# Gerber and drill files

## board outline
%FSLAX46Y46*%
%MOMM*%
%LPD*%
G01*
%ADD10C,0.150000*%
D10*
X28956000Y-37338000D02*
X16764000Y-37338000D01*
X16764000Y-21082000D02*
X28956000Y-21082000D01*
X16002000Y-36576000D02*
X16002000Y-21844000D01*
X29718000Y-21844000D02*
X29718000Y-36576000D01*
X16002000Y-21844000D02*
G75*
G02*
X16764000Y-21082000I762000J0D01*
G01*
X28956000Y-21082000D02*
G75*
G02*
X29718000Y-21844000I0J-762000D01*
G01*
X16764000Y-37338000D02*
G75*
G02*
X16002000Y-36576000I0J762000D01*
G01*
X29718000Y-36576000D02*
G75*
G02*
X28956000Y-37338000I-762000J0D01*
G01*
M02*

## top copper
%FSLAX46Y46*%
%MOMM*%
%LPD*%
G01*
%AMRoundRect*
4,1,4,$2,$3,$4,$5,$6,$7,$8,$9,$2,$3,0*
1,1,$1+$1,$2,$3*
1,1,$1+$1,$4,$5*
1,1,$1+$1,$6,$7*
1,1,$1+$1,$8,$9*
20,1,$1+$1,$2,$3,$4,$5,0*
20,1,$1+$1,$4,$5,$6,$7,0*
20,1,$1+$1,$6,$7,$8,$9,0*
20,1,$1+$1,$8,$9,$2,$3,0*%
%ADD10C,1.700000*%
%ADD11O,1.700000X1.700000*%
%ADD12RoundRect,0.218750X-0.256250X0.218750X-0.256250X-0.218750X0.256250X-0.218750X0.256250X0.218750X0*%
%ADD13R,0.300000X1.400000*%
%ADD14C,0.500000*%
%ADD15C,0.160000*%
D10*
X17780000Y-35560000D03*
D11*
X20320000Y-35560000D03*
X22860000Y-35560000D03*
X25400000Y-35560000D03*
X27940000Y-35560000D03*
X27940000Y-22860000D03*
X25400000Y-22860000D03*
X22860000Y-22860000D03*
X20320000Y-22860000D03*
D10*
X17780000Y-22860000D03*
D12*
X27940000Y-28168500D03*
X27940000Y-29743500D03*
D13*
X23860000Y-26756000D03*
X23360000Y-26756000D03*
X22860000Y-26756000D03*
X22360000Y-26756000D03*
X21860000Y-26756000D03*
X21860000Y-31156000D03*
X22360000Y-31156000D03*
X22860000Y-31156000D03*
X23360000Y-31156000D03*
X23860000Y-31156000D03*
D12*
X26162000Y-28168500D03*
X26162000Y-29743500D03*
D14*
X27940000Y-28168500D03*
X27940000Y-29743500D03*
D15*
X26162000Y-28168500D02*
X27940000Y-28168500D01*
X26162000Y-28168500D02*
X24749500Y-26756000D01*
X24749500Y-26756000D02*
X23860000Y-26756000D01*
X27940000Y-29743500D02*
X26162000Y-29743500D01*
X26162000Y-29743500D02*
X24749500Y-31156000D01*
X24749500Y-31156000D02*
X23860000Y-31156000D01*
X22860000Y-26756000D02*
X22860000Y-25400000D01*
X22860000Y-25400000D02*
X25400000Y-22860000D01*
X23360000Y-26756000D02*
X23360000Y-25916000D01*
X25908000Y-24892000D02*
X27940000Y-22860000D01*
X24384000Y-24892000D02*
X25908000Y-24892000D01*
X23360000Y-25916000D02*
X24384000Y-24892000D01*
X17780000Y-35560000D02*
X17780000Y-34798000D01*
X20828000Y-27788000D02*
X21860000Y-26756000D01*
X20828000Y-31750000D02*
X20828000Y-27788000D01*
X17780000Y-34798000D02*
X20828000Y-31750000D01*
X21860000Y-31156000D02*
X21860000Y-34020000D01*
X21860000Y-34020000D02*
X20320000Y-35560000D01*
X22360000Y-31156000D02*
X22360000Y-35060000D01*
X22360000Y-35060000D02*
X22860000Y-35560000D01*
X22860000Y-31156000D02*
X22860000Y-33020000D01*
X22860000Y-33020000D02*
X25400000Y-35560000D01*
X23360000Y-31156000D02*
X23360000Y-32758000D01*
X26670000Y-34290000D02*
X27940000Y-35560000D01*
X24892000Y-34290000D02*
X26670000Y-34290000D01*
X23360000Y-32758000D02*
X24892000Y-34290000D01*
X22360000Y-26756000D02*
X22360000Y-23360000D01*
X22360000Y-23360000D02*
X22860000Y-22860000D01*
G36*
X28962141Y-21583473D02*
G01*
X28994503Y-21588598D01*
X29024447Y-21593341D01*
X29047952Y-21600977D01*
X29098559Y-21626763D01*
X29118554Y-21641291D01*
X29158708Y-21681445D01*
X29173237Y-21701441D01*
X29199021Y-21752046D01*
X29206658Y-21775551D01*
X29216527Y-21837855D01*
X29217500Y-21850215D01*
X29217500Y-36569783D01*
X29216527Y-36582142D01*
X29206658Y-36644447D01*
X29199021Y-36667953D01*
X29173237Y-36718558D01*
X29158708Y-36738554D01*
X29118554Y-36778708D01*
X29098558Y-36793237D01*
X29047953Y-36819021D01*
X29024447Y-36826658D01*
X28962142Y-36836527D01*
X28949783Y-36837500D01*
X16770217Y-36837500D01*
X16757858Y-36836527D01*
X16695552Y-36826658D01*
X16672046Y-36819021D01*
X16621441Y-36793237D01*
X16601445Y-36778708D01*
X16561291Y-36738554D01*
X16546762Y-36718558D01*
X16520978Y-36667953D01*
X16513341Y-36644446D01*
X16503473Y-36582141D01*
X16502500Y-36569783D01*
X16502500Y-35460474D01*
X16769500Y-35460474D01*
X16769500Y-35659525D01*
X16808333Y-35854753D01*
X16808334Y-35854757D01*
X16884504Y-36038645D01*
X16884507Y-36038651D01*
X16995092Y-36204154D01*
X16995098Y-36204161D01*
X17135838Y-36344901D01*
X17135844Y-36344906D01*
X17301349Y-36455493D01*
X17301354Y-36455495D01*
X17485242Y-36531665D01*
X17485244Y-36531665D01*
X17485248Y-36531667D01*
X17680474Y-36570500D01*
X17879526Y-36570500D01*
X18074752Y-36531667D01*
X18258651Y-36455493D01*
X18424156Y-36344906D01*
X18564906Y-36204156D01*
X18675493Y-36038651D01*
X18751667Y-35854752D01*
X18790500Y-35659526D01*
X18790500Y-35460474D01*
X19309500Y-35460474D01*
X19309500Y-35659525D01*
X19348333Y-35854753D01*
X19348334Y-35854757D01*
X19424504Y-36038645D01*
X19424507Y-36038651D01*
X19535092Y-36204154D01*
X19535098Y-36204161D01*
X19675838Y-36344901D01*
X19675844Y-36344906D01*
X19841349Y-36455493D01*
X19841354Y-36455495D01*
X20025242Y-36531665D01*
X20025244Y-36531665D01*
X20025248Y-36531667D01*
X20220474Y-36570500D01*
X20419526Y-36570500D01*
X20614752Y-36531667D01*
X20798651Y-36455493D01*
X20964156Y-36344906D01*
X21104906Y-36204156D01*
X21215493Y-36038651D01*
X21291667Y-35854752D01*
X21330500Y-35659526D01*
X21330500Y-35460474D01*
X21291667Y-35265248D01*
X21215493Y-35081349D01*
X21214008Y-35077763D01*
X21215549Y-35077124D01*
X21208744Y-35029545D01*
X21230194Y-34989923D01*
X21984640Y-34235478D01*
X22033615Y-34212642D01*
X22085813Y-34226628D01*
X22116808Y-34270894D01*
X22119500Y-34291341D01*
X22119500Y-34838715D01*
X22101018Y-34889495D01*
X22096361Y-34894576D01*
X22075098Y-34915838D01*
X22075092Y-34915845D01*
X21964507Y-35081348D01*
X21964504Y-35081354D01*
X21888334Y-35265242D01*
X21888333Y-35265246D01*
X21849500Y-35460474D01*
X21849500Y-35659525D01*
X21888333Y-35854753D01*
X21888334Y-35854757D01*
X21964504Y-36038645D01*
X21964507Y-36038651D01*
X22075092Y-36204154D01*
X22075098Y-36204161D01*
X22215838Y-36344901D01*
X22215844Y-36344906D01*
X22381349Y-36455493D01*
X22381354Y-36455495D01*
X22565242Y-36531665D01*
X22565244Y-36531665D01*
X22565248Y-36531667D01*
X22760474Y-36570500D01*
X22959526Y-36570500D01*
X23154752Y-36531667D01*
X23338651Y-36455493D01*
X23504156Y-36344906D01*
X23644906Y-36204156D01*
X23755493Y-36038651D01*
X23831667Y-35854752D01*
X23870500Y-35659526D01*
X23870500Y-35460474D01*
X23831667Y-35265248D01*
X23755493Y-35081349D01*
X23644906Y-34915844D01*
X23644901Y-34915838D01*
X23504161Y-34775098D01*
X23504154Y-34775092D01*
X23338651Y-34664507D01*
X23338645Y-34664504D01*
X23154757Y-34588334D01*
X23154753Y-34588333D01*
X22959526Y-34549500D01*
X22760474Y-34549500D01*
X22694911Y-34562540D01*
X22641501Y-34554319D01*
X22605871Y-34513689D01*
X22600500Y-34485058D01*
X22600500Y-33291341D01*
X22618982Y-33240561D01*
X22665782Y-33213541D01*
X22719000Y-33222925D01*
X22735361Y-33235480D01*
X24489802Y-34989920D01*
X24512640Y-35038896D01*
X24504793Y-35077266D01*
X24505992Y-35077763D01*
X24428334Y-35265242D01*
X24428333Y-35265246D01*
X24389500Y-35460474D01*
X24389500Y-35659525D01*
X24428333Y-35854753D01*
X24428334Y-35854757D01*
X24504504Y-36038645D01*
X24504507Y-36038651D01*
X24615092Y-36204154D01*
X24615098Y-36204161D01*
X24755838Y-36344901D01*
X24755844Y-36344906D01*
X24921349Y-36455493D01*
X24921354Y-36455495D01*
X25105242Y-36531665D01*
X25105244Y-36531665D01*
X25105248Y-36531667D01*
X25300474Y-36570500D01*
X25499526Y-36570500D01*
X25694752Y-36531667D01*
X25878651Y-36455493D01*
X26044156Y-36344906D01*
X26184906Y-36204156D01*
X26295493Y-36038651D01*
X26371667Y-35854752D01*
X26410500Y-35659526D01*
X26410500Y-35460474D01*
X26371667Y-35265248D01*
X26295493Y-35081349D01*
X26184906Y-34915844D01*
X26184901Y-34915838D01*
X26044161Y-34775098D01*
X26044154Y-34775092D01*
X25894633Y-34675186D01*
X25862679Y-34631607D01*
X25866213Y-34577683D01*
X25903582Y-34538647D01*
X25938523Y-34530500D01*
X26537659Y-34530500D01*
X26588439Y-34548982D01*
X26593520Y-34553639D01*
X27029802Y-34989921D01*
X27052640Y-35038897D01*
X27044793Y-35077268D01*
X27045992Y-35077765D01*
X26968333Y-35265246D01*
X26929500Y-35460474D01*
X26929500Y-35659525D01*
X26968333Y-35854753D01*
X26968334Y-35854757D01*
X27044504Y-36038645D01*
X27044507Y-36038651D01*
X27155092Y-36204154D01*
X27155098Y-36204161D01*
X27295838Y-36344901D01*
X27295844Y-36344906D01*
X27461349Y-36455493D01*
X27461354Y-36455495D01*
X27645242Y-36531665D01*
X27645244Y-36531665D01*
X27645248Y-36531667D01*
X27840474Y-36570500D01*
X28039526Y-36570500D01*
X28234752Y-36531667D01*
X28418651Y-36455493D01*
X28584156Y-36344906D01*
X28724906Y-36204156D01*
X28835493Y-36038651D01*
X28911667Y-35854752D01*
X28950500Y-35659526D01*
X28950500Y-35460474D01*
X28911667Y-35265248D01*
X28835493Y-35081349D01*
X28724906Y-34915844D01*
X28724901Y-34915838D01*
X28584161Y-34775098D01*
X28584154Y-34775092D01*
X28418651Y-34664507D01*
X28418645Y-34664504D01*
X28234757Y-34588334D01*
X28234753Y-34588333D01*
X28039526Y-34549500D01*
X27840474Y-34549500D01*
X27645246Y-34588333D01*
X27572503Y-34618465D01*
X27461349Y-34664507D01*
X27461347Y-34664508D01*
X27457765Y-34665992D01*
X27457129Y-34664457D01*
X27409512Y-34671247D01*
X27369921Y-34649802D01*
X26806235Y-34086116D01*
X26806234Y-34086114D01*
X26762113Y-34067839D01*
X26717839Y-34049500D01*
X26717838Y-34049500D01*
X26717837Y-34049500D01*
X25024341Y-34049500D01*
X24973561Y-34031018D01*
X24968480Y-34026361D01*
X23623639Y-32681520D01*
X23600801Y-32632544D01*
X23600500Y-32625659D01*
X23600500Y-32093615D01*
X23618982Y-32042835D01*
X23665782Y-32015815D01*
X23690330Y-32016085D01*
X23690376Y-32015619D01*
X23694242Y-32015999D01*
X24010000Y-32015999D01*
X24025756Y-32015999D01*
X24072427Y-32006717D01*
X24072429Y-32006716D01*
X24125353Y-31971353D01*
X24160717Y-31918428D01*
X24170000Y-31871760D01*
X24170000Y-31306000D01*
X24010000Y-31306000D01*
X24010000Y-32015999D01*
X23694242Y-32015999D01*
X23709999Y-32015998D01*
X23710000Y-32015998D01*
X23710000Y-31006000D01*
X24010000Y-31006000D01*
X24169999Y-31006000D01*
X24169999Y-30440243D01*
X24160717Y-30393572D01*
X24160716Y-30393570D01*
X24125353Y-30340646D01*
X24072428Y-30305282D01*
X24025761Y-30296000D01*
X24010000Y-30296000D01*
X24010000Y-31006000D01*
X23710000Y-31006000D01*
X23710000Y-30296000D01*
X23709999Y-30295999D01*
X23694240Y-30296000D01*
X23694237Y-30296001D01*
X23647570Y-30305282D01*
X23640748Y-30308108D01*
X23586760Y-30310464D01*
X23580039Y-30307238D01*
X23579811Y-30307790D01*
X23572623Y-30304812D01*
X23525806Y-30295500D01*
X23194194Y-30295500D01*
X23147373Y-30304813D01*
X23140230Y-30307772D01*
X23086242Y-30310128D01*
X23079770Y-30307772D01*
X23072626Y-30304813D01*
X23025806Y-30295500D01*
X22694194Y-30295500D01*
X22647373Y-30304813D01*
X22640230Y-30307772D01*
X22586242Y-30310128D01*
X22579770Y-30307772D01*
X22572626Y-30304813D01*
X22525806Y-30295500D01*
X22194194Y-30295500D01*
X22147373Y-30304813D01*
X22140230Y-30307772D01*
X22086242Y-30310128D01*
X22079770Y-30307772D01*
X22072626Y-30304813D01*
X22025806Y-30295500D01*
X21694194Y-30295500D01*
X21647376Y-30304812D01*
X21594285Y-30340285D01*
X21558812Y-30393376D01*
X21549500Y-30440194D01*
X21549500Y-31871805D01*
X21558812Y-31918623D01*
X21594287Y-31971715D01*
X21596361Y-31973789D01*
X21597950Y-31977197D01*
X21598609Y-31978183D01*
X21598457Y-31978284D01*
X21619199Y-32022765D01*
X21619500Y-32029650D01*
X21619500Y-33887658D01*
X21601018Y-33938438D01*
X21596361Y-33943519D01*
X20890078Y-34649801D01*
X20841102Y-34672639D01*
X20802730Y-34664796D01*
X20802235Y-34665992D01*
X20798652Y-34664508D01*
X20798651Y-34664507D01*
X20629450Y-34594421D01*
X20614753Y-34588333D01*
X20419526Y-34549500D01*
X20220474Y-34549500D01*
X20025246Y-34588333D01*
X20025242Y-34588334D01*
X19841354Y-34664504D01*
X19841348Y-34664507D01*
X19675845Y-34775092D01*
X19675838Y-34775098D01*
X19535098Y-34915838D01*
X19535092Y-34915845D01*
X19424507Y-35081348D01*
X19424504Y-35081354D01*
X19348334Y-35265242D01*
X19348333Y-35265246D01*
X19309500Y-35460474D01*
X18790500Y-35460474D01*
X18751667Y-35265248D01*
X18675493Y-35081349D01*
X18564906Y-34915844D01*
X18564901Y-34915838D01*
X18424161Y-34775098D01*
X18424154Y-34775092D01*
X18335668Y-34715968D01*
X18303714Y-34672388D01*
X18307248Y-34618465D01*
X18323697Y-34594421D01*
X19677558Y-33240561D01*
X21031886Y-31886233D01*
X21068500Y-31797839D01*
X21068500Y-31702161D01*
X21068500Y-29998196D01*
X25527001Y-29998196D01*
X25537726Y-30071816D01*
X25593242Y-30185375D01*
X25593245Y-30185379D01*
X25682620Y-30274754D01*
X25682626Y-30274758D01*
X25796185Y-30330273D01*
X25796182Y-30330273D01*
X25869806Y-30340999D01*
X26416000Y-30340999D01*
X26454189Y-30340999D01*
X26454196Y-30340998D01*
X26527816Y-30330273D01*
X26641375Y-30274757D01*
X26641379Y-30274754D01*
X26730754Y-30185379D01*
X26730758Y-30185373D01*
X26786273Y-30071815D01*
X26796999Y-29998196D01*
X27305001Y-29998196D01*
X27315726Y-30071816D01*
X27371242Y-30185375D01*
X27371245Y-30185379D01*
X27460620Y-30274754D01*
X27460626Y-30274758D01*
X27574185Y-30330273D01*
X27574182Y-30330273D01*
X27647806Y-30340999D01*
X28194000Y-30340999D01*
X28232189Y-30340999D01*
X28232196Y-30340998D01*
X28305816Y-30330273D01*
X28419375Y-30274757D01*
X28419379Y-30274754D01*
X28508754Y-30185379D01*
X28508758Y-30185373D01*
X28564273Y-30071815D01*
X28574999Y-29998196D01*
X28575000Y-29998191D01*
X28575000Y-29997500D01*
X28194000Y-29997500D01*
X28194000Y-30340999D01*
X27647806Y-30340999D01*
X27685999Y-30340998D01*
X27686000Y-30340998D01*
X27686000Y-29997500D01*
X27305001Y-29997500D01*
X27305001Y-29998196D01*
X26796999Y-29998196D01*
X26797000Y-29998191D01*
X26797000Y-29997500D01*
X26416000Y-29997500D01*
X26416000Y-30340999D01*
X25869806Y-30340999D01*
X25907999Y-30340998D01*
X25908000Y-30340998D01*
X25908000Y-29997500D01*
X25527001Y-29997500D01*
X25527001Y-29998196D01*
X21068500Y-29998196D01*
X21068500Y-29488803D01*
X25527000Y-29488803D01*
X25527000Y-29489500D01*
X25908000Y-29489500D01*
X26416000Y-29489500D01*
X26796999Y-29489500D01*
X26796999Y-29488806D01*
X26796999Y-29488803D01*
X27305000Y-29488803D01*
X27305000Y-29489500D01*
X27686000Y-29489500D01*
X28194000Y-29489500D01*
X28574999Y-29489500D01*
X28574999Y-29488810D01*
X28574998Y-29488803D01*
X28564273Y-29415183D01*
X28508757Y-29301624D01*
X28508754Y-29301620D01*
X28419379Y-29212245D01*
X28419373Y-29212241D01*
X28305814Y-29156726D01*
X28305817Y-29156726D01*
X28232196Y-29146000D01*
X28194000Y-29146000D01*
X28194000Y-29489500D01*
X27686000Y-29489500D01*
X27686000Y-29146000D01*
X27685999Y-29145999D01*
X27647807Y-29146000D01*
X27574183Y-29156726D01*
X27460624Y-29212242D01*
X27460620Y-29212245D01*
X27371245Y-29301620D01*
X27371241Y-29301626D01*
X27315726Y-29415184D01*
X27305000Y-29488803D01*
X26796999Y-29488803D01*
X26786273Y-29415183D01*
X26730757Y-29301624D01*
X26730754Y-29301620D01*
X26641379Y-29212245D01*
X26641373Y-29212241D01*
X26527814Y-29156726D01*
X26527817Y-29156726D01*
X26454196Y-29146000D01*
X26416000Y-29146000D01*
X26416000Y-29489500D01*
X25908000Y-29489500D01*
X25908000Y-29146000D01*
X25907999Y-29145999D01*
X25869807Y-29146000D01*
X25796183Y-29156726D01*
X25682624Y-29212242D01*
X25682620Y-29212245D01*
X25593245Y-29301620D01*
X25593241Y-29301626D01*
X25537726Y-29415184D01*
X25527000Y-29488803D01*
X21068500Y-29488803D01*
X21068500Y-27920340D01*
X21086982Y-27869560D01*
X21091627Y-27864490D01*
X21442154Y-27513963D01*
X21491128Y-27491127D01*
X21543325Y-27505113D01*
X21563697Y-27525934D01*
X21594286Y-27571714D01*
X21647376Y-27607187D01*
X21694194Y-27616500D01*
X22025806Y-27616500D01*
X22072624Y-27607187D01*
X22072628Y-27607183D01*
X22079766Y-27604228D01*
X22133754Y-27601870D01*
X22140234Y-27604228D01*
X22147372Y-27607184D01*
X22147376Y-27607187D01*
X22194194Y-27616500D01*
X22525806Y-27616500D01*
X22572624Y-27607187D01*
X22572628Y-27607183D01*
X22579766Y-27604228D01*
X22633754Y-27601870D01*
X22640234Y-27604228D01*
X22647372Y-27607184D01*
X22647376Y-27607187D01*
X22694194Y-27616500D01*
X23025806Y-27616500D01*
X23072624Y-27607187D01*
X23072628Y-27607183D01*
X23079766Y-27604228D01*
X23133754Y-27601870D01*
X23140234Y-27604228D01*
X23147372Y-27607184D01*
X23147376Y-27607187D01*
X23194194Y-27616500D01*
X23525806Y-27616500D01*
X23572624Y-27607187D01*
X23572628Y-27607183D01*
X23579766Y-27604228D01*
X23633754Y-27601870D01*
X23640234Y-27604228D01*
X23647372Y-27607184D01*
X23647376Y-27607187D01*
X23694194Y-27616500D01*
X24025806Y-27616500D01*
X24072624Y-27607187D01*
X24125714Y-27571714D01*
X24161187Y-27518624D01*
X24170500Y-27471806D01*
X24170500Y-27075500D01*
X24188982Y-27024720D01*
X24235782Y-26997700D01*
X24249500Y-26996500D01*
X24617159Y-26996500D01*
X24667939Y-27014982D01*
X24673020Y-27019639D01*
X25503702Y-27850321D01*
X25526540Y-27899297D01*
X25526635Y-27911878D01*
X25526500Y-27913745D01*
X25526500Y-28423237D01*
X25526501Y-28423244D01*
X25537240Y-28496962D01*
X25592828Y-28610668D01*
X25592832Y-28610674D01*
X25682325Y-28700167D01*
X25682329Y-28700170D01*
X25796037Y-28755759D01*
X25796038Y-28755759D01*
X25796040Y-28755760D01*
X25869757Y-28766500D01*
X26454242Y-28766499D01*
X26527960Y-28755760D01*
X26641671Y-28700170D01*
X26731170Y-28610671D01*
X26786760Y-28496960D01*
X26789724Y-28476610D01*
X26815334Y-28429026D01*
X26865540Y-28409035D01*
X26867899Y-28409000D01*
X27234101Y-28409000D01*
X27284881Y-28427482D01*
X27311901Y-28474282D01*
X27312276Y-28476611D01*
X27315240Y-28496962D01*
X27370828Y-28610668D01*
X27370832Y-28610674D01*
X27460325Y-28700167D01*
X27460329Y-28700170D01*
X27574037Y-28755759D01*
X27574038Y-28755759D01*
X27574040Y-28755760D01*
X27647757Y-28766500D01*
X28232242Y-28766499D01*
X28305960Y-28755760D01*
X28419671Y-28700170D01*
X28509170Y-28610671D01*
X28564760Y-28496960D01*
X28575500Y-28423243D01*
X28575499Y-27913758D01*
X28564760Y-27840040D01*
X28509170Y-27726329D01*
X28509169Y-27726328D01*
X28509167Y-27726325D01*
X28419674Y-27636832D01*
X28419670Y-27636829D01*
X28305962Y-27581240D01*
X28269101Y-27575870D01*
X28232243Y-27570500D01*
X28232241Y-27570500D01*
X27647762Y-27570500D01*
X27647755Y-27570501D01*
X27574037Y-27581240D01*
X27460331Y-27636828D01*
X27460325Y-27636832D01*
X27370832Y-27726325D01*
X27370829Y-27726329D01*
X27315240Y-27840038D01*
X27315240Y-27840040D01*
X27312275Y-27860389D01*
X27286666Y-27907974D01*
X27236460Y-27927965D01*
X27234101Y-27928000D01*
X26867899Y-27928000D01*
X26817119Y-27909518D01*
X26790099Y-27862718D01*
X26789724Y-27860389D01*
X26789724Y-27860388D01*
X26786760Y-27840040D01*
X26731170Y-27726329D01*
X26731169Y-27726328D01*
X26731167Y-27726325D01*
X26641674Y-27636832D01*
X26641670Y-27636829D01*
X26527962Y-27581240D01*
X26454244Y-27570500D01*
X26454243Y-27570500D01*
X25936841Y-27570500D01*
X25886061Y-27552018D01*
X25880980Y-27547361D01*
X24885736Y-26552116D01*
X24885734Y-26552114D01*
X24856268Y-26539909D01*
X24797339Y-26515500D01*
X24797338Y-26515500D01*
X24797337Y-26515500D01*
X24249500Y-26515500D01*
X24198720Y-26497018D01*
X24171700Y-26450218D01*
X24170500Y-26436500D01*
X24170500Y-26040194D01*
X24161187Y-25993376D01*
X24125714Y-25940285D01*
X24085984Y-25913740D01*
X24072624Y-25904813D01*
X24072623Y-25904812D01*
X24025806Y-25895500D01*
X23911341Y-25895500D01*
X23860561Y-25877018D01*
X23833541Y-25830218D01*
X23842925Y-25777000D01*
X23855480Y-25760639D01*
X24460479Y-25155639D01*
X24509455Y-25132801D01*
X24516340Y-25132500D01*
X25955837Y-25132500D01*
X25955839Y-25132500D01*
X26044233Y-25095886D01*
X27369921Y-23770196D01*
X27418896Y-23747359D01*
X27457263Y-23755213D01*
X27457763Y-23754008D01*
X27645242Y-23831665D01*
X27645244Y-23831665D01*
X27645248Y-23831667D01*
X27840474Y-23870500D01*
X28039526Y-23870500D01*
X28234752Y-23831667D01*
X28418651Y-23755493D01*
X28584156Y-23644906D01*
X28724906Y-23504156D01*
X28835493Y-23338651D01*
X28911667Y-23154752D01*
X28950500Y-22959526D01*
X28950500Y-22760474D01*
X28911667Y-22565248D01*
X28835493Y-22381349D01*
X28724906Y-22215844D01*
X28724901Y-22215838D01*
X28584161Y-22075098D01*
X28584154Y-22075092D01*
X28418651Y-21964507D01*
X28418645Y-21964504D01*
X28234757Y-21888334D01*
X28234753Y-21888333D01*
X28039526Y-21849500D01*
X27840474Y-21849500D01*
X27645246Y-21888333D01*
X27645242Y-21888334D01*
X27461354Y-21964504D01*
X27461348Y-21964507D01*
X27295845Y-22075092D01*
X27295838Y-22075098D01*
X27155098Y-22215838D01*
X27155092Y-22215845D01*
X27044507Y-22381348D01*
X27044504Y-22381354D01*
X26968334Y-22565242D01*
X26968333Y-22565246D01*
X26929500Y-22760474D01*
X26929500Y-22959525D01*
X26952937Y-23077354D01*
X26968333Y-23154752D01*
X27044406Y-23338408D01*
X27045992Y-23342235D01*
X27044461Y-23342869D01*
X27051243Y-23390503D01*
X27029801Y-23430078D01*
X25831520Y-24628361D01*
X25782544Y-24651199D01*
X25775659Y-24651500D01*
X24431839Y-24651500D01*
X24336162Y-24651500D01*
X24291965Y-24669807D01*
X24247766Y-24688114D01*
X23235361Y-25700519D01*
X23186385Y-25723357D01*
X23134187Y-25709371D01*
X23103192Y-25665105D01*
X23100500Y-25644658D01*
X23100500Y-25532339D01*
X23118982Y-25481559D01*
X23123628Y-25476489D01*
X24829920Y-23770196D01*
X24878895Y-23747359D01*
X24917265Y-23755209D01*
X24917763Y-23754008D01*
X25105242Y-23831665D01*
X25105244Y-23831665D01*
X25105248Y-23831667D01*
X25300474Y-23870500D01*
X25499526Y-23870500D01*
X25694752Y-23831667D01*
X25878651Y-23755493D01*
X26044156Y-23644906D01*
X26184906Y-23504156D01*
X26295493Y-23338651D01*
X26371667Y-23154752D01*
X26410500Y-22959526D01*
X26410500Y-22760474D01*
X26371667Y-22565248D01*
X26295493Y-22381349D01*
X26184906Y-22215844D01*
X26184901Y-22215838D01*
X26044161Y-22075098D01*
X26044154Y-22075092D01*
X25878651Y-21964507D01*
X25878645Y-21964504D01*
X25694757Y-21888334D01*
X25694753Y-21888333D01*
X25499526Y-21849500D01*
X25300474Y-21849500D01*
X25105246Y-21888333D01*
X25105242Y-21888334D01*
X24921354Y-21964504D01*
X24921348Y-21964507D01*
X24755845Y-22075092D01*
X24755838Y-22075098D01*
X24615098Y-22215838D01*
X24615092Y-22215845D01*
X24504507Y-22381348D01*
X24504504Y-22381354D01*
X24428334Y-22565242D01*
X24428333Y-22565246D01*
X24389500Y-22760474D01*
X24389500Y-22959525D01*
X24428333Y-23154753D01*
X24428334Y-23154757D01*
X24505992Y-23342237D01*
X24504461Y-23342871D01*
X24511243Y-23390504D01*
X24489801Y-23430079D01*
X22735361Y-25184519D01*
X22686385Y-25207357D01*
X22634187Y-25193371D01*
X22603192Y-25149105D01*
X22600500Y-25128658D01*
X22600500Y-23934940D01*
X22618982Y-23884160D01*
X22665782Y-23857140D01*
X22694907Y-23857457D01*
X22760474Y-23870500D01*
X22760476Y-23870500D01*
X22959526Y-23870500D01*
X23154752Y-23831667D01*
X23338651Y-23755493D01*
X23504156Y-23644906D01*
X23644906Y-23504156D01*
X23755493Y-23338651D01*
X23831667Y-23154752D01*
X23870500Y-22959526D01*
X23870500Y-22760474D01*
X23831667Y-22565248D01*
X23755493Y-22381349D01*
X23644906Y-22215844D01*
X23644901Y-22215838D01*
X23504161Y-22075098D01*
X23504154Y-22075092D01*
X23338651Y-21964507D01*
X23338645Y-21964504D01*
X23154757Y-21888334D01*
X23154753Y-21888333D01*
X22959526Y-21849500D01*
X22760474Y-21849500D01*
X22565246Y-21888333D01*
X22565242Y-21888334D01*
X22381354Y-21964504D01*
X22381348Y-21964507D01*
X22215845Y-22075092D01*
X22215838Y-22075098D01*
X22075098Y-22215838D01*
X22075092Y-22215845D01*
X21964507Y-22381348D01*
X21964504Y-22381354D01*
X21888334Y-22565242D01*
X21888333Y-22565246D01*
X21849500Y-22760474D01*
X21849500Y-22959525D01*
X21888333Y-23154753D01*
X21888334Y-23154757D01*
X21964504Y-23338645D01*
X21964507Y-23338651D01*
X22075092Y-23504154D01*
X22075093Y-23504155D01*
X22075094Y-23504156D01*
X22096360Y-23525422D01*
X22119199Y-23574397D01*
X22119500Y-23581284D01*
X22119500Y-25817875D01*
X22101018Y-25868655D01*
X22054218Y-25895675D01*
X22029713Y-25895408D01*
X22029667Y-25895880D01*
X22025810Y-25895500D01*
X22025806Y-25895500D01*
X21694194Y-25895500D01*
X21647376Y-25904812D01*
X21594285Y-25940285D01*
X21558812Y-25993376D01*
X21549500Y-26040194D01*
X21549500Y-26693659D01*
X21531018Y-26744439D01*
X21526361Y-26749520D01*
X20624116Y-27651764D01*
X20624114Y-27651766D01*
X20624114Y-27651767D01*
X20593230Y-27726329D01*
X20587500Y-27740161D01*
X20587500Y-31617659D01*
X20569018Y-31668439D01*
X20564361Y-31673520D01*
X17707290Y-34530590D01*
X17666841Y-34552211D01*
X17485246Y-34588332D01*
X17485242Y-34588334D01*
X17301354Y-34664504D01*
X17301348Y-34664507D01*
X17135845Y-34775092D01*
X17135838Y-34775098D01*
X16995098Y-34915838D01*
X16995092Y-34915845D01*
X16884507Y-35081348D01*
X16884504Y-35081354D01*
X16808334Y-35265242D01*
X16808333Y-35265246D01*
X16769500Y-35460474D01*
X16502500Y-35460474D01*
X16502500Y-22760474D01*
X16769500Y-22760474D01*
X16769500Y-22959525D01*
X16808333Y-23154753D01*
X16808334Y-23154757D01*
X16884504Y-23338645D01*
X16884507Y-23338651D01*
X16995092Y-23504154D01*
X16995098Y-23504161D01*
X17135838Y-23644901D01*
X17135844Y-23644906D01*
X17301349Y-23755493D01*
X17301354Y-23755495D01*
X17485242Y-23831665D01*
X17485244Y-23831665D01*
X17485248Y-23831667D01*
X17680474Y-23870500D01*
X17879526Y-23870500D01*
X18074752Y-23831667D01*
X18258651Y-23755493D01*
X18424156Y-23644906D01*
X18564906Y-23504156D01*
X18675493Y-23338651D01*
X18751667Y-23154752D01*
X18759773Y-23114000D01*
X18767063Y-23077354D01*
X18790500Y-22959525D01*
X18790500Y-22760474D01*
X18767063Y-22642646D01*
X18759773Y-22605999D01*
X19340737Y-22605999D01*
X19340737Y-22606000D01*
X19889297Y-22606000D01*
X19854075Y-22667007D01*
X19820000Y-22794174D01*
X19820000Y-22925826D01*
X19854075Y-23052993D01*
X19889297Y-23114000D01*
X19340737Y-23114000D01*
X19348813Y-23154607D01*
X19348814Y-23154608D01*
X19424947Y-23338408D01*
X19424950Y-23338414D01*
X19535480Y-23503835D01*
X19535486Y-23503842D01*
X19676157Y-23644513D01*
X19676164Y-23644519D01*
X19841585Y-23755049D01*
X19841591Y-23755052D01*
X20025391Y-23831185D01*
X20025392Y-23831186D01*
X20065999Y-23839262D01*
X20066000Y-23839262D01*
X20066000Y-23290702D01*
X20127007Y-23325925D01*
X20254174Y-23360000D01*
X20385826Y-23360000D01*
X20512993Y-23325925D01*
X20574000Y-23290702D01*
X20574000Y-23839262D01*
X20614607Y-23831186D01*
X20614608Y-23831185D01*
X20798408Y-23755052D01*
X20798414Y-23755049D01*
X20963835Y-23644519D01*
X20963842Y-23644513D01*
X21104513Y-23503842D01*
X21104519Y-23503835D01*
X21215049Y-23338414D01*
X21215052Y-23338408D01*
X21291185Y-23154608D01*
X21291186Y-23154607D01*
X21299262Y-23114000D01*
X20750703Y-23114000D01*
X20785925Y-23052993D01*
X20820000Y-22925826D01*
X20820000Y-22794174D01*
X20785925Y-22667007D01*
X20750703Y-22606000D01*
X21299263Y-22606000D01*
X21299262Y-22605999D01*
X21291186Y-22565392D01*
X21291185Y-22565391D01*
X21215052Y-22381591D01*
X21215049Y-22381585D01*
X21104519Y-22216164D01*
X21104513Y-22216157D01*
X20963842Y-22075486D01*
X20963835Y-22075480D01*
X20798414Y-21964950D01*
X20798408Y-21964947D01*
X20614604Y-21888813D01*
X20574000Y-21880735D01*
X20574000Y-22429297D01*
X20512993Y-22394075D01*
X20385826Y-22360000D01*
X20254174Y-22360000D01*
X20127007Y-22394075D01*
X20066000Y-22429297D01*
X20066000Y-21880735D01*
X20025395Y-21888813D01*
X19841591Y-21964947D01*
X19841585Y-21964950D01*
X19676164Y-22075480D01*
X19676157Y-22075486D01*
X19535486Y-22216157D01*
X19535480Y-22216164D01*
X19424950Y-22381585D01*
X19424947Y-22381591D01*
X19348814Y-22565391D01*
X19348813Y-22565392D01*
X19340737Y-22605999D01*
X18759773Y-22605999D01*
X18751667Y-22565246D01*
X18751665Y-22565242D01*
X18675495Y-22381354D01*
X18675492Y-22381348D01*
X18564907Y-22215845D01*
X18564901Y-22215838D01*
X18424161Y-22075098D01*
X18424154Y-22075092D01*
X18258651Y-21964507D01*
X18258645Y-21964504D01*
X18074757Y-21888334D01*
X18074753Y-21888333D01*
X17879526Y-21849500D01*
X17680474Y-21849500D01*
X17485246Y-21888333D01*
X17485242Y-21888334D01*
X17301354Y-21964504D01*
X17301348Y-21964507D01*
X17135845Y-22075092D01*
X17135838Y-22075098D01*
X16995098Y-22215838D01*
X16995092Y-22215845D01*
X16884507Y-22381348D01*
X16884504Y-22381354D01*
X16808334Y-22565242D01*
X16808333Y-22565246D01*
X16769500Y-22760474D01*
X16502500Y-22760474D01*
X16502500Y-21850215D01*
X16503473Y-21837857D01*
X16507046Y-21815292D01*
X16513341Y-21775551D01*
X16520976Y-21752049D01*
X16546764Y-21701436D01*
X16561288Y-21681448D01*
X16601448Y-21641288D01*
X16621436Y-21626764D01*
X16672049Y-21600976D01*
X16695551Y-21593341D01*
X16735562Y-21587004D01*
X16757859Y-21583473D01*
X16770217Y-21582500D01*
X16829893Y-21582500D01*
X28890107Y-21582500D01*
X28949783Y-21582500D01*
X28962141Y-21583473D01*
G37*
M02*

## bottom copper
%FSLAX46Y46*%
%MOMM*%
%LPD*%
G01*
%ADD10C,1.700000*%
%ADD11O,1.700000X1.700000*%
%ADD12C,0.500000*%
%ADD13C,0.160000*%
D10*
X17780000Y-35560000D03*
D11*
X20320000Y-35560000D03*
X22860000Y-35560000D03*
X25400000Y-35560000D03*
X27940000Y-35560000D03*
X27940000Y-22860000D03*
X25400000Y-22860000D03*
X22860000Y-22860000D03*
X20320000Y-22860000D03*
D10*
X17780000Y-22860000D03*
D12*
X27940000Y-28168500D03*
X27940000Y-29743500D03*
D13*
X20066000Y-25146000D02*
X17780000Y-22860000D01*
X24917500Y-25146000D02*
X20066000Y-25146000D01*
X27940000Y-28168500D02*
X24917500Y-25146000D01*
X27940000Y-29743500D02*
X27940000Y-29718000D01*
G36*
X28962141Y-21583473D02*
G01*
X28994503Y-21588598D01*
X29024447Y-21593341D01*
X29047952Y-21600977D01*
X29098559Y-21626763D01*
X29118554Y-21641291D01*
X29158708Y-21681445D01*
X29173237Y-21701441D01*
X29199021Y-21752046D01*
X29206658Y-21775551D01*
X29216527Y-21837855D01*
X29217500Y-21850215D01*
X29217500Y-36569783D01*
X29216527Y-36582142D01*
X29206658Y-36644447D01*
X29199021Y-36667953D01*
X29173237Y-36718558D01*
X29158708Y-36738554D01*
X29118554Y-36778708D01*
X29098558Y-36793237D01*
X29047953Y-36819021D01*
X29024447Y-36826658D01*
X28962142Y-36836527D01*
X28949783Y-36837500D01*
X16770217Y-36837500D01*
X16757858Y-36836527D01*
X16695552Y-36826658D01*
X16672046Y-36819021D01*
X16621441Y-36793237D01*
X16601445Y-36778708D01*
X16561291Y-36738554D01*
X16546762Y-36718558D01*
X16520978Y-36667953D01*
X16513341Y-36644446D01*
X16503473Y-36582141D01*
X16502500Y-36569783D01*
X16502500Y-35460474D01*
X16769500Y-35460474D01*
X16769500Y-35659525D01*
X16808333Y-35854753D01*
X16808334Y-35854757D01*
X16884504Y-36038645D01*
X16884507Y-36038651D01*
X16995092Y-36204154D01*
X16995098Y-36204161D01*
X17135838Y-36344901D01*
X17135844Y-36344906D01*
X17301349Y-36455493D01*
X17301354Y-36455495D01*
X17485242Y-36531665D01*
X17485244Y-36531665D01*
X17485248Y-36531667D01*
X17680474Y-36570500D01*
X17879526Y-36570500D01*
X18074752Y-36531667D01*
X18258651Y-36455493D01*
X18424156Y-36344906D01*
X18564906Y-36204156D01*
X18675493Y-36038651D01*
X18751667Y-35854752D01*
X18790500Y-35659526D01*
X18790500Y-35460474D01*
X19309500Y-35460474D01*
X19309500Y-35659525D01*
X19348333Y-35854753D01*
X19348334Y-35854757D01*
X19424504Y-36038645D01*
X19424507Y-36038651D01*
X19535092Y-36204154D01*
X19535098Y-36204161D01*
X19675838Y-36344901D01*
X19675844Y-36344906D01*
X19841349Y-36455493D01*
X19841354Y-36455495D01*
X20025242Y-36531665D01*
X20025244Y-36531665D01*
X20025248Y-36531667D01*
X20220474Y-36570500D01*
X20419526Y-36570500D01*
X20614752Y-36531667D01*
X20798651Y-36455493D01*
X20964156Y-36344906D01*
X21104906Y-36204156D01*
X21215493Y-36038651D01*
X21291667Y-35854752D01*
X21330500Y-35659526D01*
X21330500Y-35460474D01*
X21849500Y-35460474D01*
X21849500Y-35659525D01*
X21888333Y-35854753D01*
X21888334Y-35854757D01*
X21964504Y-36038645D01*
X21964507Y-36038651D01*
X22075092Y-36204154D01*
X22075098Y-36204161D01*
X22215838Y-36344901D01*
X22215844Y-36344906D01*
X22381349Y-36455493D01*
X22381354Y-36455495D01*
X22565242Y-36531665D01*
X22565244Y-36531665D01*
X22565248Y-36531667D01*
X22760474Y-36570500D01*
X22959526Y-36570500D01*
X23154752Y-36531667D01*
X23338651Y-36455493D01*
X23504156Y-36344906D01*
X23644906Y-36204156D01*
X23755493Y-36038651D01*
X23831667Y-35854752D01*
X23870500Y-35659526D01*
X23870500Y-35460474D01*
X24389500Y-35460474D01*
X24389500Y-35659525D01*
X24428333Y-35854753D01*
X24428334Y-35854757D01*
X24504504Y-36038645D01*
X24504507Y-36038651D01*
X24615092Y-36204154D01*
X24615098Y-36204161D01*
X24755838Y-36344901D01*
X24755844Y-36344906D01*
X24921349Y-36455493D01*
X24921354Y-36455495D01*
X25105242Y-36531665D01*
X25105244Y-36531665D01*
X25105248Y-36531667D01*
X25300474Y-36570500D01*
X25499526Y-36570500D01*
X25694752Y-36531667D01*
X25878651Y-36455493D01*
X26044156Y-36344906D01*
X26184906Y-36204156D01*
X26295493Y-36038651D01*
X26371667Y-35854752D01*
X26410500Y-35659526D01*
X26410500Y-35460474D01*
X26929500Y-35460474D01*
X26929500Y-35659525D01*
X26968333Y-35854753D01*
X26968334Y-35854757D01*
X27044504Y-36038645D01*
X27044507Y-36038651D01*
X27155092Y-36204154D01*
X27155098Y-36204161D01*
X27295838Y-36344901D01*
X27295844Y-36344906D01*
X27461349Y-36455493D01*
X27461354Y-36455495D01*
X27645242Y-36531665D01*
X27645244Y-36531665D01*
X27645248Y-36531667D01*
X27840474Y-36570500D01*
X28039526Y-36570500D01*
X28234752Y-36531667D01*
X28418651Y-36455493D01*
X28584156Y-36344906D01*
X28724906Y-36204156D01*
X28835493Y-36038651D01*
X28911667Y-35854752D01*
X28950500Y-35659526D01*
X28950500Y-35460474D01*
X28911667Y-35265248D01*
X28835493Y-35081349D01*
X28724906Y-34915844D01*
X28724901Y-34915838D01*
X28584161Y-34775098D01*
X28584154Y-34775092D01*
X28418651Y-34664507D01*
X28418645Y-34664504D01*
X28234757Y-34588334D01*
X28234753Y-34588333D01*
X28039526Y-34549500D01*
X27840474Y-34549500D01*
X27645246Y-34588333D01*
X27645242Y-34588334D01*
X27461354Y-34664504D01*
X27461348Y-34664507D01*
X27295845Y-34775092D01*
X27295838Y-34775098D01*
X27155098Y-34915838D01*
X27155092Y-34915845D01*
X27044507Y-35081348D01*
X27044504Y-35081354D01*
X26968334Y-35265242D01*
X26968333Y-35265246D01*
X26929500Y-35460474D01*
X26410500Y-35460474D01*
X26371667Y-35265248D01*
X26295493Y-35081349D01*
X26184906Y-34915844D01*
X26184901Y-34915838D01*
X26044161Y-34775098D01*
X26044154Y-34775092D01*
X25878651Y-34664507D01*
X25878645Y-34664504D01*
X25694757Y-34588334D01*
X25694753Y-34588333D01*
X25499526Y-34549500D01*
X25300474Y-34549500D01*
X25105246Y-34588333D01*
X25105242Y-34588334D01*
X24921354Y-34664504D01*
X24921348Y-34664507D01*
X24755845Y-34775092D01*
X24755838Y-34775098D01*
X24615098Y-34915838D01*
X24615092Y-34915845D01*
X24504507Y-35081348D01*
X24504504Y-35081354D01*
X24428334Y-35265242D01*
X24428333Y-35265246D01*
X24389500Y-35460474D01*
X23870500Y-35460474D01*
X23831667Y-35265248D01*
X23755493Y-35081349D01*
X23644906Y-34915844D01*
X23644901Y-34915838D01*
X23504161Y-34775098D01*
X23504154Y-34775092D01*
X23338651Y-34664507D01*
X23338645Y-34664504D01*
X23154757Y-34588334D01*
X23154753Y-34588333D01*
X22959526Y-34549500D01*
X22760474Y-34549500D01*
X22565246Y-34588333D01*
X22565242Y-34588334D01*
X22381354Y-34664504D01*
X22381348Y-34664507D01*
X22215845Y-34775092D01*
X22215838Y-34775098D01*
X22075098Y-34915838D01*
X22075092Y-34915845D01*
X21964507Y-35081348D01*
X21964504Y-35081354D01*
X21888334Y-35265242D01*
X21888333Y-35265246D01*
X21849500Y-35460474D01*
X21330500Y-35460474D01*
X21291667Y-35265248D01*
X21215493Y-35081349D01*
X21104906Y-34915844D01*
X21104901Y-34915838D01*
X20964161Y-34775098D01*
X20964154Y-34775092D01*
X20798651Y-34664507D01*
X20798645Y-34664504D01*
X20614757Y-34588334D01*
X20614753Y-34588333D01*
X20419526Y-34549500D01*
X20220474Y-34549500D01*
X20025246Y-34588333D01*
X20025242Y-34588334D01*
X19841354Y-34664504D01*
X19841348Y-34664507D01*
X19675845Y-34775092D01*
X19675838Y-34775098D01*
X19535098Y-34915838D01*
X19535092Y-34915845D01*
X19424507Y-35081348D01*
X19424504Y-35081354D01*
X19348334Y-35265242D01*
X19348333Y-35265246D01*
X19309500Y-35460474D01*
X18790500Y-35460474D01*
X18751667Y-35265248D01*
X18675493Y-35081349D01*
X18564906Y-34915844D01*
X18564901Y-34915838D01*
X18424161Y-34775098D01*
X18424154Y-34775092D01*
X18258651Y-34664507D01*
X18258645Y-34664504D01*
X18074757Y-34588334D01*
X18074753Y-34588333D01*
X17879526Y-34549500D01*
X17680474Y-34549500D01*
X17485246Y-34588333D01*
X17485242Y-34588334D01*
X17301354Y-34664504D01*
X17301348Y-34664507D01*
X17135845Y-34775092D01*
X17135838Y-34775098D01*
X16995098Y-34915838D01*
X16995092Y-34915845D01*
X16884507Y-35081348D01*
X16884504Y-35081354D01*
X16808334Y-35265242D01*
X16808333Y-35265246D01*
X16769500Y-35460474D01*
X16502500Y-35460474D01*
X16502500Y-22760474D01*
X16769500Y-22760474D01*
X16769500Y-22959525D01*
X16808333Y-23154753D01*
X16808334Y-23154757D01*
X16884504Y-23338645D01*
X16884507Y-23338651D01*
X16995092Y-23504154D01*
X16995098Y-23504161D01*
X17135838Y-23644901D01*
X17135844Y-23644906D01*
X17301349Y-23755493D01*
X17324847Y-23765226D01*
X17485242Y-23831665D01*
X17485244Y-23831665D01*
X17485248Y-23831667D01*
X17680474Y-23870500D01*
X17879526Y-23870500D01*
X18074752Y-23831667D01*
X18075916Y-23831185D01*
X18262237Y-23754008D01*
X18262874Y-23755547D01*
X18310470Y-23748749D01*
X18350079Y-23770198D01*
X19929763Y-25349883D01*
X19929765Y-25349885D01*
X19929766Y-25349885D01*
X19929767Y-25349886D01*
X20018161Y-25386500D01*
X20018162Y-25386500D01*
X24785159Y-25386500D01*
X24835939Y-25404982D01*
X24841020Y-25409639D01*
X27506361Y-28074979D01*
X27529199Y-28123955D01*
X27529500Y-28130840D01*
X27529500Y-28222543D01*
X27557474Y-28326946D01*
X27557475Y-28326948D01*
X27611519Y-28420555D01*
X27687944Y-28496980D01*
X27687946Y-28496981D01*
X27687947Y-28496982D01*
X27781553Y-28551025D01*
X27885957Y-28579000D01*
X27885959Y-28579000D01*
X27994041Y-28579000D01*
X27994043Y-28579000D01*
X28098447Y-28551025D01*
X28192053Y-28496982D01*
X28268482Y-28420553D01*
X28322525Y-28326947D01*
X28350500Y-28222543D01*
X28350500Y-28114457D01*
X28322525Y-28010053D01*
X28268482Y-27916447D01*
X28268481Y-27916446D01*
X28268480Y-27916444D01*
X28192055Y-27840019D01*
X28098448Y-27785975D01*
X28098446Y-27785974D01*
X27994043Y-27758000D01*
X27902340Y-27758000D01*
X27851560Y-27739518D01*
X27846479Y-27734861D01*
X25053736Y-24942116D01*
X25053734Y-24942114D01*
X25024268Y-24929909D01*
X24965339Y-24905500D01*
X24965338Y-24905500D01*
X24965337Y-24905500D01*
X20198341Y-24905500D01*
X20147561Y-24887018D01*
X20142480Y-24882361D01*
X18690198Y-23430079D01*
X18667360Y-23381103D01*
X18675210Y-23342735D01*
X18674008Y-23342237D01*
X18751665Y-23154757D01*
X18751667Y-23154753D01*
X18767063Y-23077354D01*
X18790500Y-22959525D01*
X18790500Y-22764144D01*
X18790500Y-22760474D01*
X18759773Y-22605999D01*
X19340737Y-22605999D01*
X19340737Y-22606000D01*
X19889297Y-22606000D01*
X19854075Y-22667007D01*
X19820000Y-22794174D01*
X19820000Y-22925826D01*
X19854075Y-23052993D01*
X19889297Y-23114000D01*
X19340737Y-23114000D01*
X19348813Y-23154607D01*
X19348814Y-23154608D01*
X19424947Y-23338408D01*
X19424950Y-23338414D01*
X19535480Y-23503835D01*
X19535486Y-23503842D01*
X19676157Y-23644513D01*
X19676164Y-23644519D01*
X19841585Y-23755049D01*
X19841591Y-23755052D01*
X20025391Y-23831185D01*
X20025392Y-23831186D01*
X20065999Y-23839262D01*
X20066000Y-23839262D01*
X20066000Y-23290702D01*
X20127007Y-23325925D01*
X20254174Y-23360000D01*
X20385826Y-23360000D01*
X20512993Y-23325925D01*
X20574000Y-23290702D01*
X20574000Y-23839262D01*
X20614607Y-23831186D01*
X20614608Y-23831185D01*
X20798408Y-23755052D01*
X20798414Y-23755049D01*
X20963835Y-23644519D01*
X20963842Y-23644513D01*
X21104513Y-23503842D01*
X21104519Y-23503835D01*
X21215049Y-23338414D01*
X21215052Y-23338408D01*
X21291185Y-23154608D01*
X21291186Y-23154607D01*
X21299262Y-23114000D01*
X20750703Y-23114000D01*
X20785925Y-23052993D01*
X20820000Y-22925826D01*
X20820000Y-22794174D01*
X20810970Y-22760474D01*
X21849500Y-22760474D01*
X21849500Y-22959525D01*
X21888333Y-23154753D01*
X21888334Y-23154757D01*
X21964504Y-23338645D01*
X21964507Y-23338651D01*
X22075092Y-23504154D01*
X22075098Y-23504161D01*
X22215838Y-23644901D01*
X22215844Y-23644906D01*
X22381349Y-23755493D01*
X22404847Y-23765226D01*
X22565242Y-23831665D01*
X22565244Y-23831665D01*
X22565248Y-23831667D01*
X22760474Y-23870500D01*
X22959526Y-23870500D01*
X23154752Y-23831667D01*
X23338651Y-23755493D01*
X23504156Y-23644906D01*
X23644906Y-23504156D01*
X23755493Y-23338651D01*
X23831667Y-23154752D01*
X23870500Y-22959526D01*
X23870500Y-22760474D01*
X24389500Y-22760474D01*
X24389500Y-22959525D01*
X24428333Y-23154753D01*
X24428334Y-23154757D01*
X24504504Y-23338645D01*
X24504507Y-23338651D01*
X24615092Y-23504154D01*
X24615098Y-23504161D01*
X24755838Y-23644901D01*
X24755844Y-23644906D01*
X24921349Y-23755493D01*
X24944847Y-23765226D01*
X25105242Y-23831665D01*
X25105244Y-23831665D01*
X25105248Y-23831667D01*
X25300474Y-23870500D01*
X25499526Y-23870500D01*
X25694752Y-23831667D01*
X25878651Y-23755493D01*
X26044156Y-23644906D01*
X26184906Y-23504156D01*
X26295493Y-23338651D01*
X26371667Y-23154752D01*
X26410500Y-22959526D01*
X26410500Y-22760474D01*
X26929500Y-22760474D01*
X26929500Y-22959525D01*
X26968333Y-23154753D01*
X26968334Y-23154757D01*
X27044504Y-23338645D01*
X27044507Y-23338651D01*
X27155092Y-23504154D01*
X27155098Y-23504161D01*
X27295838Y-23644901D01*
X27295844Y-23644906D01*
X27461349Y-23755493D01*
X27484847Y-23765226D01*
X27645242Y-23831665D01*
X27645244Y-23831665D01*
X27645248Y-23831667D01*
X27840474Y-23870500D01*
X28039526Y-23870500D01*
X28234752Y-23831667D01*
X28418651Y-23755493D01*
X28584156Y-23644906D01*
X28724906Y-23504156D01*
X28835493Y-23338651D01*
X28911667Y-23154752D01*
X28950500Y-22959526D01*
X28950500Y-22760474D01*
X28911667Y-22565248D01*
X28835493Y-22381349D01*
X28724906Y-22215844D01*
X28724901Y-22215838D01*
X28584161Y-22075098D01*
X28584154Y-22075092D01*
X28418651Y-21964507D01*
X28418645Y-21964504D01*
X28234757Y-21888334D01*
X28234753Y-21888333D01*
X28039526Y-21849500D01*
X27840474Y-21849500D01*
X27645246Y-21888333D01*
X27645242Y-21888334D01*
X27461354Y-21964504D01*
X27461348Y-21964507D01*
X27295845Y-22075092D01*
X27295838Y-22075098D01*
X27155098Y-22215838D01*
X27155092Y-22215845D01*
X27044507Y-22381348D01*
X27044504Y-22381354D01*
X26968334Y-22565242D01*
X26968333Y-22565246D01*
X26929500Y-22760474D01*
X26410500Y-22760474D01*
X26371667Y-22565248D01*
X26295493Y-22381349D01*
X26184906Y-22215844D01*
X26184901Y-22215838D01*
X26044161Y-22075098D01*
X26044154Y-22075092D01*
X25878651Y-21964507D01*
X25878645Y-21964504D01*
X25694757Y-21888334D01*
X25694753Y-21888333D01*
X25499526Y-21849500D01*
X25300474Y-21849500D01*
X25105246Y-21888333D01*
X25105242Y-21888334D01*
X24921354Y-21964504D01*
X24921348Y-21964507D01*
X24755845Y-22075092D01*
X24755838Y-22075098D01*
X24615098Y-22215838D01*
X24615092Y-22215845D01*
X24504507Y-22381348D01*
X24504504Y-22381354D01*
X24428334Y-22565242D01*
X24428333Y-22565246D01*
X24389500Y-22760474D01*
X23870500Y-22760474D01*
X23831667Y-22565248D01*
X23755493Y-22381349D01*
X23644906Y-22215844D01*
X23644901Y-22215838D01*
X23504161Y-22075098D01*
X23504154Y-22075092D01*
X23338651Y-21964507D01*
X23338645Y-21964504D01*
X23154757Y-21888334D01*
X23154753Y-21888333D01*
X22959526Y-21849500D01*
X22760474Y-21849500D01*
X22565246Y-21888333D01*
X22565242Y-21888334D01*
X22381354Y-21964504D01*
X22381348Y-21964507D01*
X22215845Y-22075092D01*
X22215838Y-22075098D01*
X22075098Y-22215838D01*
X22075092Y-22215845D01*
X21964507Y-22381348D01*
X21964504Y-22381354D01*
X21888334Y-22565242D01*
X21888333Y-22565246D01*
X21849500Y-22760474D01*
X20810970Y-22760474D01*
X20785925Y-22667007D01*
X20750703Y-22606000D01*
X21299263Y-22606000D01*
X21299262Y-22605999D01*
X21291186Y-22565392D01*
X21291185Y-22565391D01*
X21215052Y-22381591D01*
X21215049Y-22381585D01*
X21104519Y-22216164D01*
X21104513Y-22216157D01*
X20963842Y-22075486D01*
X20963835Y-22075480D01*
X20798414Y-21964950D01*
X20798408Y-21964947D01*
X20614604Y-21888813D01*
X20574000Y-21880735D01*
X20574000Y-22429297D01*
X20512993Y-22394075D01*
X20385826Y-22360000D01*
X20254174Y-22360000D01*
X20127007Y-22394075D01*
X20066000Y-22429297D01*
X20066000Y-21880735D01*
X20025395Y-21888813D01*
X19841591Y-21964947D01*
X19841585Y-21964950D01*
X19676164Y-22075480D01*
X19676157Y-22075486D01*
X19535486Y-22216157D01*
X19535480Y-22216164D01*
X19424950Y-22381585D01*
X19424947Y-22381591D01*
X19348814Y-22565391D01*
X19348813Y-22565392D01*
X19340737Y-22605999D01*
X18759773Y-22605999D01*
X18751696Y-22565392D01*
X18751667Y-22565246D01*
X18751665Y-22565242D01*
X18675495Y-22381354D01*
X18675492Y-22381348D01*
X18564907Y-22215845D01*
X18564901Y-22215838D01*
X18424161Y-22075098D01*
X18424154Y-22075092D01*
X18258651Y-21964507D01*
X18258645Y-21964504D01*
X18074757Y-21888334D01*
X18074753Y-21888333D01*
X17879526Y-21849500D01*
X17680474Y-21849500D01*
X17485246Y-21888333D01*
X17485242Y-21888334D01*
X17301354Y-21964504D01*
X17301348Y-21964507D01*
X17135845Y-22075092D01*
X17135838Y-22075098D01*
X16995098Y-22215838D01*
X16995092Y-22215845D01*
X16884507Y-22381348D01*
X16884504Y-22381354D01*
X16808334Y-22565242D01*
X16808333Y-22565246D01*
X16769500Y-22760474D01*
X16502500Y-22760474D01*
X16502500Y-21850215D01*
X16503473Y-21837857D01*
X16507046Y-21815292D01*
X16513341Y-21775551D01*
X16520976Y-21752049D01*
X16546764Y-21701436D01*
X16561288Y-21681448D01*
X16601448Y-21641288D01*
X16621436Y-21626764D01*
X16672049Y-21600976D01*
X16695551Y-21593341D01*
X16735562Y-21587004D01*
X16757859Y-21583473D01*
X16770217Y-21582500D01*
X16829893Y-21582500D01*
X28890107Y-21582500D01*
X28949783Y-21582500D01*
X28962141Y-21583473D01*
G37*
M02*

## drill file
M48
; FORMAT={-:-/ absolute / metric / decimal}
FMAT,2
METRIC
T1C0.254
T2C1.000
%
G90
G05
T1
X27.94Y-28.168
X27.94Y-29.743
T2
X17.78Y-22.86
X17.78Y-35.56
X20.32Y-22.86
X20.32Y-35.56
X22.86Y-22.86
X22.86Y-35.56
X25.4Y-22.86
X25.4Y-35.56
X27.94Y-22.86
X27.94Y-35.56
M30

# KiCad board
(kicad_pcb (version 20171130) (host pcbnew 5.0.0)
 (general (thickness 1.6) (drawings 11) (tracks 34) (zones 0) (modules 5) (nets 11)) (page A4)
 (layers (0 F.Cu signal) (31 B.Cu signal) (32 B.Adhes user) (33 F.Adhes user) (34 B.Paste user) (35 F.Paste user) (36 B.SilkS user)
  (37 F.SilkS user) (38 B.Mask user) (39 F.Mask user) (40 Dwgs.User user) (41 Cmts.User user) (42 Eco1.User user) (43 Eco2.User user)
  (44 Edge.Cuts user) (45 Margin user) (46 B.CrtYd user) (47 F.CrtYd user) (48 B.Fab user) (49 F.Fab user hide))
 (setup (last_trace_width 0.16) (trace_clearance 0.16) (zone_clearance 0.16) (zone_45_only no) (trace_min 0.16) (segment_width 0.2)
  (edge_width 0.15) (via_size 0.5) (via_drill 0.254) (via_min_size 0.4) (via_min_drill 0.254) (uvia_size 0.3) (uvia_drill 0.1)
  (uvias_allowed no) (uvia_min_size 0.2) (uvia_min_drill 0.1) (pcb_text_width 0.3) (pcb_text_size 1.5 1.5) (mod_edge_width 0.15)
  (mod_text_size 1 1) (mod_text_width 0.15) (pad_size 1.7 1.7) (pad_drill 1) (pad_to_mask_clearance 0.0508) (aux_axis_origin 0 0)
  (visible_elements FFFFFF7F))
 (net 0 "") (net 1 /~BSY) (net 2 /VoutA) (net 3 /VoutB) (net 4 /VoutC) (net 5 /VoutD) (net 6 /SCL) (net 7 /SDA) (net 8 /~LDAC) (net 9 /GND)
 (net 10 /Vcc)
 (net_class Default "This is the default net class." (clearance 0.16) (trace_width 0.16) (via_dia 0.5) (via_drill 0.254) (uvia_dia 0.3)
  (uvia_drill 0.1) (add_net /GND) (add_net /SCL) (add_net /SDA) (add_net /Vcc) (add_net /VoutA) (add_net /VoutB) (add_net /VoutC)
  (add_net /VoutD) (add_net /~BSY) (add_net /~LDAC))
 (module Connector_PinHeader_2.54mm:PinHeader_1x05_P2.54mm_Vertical (layer F.Cu) (at 17.78 35.56 90)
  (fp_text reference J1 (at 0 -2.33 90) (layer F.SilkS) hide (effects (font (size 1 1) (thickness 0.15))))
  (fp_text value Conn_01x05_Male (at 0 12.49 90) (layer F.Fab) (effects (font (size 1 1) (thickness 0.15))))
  (pad 1 thru_hole circle (at 0 0 90) (size 1.7 1.7) (drill 1) (layers *.Cu *.Mask) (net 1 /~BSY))
  (pad 2 thru_hole oval (at 0 2.54 90) (size 1.7 1.7) (drill 1) (layers *.Cu *.Mask) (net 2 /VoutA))
  (pad 3 thru_hole oval (at 0 5.08 90) (size 1.7 1.7) (drill 1) (layers *.Cu *.Mask) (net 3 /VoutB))
  (pad 4 thru_hole oval (at 0 7.62 90) (size 1.7 1.7) (drill 1) (layers *.Cu *.Mask) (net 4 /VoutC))
  (pad 5 thru_hole oval (at 0 10.16 90) (size 1.7 1.7) (drill 1) (layers *.Cu *.Mask) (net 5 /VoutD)))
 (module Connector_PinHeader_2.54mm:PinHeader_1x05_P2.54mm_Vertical (layer F.Cu) (at 17.78 22.86 90)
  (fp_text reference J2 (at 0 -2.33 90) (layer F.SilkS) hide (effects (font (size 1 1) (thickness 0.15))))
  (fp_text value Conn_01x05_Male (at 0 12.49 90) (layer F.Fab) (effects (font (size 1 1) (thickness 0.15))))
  (pad 5 thru_hole oval (at 0 10.16 90) (size 1.7 1.7) (drill 1) (layers *.Cu *.Mask) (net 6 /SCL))
  (pad 4 thru_hole oval (at 0 7.62 90) (size 1.7 1.7) (drill 1) (layers *.Cu *.Mask) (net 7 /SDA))
  (pad 3 thru_hole oval (at 0 5.08 90) (size 1.7 1.7) (drill 1) (layers *.Cu *.Mask) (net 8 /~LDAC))
  (pad 2 thru_hole oval (at 0 2.54 90) (size 1.7 1.7) (drill 1) (layers *.Cu *.Mask) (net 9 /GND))
  (pad 1 thru_hole circle (at 0 0 90) (size 1.7 1.7) (drill 1) (layers *.Cu *.Mask) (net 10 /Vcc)))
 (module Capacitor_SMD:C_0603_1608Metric (layer F.Cu) (at 27.94 28.956 270)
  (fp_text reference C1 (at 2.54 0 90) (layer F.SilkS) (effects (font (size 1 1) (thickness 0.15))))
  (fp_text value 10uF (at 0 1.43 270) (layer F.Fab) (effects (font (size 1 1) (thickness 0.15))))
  (pad 1 smd roundrect (at -0.7875 0 270) (size 0.875 0.95) (layers F.Cu F.Paste F.Mask) (roundrect_rratio 0.25) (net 10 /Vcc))
  (pad 2 smd roundrect (at 0.7875 0 270) (size 0.875 0.95) (layers F.Cu F.Paste F.Mask) (roundrect_rratio 0.25) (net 9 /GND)))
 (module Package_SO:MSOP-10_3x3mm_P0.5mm (layer F.Cu) (at 22.86 28.956 270)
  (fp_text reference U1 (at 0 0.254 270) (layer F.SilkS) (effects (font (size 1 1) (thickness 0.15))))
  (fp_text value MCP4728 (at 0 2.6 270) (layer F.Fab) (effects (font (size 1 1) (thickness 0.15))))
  (pad 1 smd rect (at -2.2 -1 270) (size 1.4 0.3) (layers F.Cu F.Paste F.Mask) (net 10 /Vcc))
  (pad 2 smd rect (at -2.2 -0.5 270) (size 1.4 0.3) (layers F.Cu F.Paste F.Mask) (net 6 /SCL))
  (pad 3 smd rect (at -2.2 0 270) (size 1.4 0.3) (layers F.Cu F.Paste F.Mask) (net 7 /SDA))
  (pad 4 smd rect (at -2.2 0.5 270) (size 1.4 0.3) (layers F.Cu F.Paste F.Mask) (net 8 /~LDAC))
  (pad 5 smd rect (at -2.2 1 270) (size 1.4 0.3) (layers F.Cu F.Paste F.Mask) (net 1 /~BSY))
  (pad 6 smd rect (at 2.2 1 270) (size 1.4 0.3) (layers F.Cu F.Paste F.Mask) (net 2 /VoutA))
  (pad 7 smd rect (at 2.2 0.5 270) (size 1.4 0.3) (layers F.Cu F.Paste F.Mask) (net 3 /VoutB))
  (pad 8 smd rect (at 2.2 0 270) (size 1.4 0.3) (layers F.Cu F.Paste F.Mask) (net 4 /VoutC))
  (pad 9 smd rect (at 2.2 -0.5 270) (size 1.4 0.3) (layers F.Cu F.Paste F.Mask) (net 5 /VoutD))
  (pad 10 smd rect (at 2.2 -1 270) (size 1.4 0.3) (layers F.Cu F.Paste F.Mask) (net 9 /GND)))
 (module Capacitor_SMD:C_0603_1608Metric (layer F.Cu) (at 26.162 28.956 270)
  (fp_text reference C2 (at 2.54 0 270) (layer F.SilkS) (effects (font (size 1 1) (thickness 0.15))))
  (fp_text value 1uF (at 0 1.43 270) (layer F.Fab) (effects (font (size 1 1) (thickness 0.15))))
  (pad 1 smd roundrect (at -0.7875 0 270) (size 0.875 0.95) (layers F.Cu F.Paste F.Mask) (roundrect_rratio 0.25) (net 10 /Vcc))
  (pad 2 smd roundrect (at 0.7875 0 270) (size 0.875 0.95) (layers F.Cu F.Paste F.Mask) (roundrect_rratio 0.25) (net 9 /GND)))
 (gr_line (start 28.956 37.338) (end 16.764 37.338) (angle 90) (layer Edge.Cuts) (width 0.15))
 (gr_line (start 16.764 21.082) (end 28.956 21.082) (angle 90) (layer Edge.Cuts) (width 0.15))
 (gr_line (start 16.002 36.576) (end 16.002 21.844) (angle 90) (layer Edge.Cuts) (width 0.15))
 (gr_line (start 29.718 21.844) (end 29.718 36.576) (angle 90) (layer Edge.Cuts) (width 0.15))
 (gr_arc (start 16.764 21.844) (end 16.002 21.844) (angle 90) (layer Edge.Cuts) (width 0.15))
 (gr_arc (start 28.956 21.844) (end 28.956 21.082) (angle 90) (layer Edge.Cuts) (width 0.15))
 (gr_arc (start 16.764 36.576) (end 16.764 37.338) (angle 90) (layer Edge.Cuts) (width 0.15))
 (gr_arc (start 28.956 36.576) (end 29.718 36.576) (angle 90) (layer Edge.Cuts) (width 0.15))
 (segment (start 26.162 28.1685) (end 27.94 28.1685) (width 0.16) (layer F.Cu) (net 10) (status C00000))
 (segment (start 20.066 25.146) (end 17.78 22.86) (width 0.16) (layer B.Cu) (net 10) (status 800000))
 (segment (start 24.9175 25.146) (end 20.066 25.146) (width 0.16) (layer B.Cu) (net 10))
 (segment (start 27.94 28.1685) (end 24.9175 25.146) (width 0.16) (layer B.Cu) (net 10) (status 400000))
 (via (at 27.94 28.1685) (size 0.5) (drill 0.254) (layers F.Cu B.Cu) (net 10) (status C00000))
 (segment (start 26.162 28.1685) (end 24.7495 26.756) (width 0.16) (layer F.Cu) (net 10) (status 400000))
 (segment (start 24.7495 26.756) (end 23.86 26.756) (width 0.16) (layer F.Cu) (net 10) (status 800000))
 (segment (start 27.94 29.7435) (end 26.162 29.7435) (width 0.16) (layer F.Cu) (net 9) (status C00000))
 (segment (start 26.162 29.7435) (end 24.7495 31.156) (width 0.16) (layer F.Cu) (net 9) (status 400000))
 (segment (start 24.7495 31.156) (end 23.86 31.156) (width 0.16) (layer F.Cu) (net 9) (status 800000))
 (via (at 27.94 29.7435) (size 0.5) (drill 0.254) (layers F.Cu B.Cu) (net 9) (status C00000))
 (segment (start 27.94 29.7435) (end 27.94 29.718) (width 0.16) (layer B.Cu) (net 9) (status 400000))
 (segment (start 22.86 26.756) (end 22.86 25.4) (width 0.16) (layer F.Cu) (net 7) (status 400000))
 (segment (start 22.86 25.4) (end 25.4 22.86) (width 0.16) (layer F.Cu) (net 7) (status 800000))
 (segment (start 23.36 26.756) (end 23.36 25.916) (width 0.16) (layer F.Cu) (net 6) (status 400000))
 (segment (start 25.908 24.892) (end 27.94 22.86) (width 0.16) (layer F.Cu) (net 6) (status 800000))
 (segment (start 24.384 24.892) (end 25.908 24.892) (width 0.16) (layer F.Cu) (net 6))
 (segment (start 23.36 25.916) (end 24.384 24.892) (width 0.16) (layer F.Cu) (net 6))
 (segment (start 17.78 35.56) (end 17.78 34.798) (width 0.16) (layer F.Cu) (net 1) (status C00000))
 (segment (start 20.828 27.788) (end 21.86 26.756) (width 0.16) (layer F.Cu) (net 1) (status 800000))
 (segment (start 20.828 31.75) (end 20.828 27.788) (width 0.16) (layer F.Cu) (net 1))
 (segment (start 17.78 34.798) (end 20.828 31.75) (width 0.16) (layer F.Cu) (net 1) (status 400000))
 (segment (start 21.86 31.156) (end 21.86 34.02) (width 0.16) (layer F.Cu) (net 2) (status 400000))
 (segment (start 21.86 34.02) (end 20.32 35.56) (width 0.16) (layer F.Cu) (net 2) (status 800000))
 (segment (start 22.36 31.156) (end 22.36 35.06) (width 0.16) (layer F.Cu) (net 3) (status C00000))
 (segment (start 22.36 35.06) (end 22.86 35.56) (width 0.16) (layer F.Cu) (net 3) (status C00000))
 (segment (start 22.86 31.156) (end 22.86 33.02) (width 0.16) (layer F.Cu) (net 4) (status 400000))
 (segment (start 22.86 33.02) (end 25.4 35.56) (width 0.16) (layer F.Cu) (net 4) (status 800000))
 (segment (start 23.36 31.156) (end 23.36 32.758) (width 0.16) (layer F.Cu) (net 5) (status 400000))
 (segment (start 26.67 34.29) (end 27.94 35.56) (width 0.16) (layer F.Cu) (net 5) (status 800000))
 (segment (start 24.892 34.29) (end 26.67 34.29) (width 0.16) (layer F.Cu) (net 5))
 (segment (start 23.36 32.758) (end 24.892 34.29) (width 0.16) (layer F.Cu) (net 5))
 (segment (start 22.36 26.756) (end 22.36 23.36) (width 0.16) (layer F.Cu) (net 8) (status C00000))
 (segment (start 22.36 23.36) (end 22.86 22.86) (width 0.16) (layer F.Cu) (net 8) (status C00000))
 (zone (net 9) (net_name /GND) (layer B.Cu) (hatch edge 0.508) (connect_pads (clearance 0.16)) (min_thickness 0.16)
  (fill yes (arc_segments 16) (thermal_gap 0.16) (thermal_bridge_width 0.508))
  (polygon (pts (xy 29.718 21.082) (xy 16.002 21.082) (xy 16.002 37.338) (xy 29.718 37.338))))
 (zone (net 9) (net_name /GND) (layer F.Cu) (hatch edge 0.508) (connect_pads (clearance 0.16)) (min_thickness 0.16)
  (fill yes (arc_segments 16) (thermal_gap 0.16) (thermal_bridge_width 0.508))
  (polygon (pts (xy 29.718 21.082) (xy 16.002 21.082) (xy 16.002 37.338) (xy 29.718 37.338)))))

